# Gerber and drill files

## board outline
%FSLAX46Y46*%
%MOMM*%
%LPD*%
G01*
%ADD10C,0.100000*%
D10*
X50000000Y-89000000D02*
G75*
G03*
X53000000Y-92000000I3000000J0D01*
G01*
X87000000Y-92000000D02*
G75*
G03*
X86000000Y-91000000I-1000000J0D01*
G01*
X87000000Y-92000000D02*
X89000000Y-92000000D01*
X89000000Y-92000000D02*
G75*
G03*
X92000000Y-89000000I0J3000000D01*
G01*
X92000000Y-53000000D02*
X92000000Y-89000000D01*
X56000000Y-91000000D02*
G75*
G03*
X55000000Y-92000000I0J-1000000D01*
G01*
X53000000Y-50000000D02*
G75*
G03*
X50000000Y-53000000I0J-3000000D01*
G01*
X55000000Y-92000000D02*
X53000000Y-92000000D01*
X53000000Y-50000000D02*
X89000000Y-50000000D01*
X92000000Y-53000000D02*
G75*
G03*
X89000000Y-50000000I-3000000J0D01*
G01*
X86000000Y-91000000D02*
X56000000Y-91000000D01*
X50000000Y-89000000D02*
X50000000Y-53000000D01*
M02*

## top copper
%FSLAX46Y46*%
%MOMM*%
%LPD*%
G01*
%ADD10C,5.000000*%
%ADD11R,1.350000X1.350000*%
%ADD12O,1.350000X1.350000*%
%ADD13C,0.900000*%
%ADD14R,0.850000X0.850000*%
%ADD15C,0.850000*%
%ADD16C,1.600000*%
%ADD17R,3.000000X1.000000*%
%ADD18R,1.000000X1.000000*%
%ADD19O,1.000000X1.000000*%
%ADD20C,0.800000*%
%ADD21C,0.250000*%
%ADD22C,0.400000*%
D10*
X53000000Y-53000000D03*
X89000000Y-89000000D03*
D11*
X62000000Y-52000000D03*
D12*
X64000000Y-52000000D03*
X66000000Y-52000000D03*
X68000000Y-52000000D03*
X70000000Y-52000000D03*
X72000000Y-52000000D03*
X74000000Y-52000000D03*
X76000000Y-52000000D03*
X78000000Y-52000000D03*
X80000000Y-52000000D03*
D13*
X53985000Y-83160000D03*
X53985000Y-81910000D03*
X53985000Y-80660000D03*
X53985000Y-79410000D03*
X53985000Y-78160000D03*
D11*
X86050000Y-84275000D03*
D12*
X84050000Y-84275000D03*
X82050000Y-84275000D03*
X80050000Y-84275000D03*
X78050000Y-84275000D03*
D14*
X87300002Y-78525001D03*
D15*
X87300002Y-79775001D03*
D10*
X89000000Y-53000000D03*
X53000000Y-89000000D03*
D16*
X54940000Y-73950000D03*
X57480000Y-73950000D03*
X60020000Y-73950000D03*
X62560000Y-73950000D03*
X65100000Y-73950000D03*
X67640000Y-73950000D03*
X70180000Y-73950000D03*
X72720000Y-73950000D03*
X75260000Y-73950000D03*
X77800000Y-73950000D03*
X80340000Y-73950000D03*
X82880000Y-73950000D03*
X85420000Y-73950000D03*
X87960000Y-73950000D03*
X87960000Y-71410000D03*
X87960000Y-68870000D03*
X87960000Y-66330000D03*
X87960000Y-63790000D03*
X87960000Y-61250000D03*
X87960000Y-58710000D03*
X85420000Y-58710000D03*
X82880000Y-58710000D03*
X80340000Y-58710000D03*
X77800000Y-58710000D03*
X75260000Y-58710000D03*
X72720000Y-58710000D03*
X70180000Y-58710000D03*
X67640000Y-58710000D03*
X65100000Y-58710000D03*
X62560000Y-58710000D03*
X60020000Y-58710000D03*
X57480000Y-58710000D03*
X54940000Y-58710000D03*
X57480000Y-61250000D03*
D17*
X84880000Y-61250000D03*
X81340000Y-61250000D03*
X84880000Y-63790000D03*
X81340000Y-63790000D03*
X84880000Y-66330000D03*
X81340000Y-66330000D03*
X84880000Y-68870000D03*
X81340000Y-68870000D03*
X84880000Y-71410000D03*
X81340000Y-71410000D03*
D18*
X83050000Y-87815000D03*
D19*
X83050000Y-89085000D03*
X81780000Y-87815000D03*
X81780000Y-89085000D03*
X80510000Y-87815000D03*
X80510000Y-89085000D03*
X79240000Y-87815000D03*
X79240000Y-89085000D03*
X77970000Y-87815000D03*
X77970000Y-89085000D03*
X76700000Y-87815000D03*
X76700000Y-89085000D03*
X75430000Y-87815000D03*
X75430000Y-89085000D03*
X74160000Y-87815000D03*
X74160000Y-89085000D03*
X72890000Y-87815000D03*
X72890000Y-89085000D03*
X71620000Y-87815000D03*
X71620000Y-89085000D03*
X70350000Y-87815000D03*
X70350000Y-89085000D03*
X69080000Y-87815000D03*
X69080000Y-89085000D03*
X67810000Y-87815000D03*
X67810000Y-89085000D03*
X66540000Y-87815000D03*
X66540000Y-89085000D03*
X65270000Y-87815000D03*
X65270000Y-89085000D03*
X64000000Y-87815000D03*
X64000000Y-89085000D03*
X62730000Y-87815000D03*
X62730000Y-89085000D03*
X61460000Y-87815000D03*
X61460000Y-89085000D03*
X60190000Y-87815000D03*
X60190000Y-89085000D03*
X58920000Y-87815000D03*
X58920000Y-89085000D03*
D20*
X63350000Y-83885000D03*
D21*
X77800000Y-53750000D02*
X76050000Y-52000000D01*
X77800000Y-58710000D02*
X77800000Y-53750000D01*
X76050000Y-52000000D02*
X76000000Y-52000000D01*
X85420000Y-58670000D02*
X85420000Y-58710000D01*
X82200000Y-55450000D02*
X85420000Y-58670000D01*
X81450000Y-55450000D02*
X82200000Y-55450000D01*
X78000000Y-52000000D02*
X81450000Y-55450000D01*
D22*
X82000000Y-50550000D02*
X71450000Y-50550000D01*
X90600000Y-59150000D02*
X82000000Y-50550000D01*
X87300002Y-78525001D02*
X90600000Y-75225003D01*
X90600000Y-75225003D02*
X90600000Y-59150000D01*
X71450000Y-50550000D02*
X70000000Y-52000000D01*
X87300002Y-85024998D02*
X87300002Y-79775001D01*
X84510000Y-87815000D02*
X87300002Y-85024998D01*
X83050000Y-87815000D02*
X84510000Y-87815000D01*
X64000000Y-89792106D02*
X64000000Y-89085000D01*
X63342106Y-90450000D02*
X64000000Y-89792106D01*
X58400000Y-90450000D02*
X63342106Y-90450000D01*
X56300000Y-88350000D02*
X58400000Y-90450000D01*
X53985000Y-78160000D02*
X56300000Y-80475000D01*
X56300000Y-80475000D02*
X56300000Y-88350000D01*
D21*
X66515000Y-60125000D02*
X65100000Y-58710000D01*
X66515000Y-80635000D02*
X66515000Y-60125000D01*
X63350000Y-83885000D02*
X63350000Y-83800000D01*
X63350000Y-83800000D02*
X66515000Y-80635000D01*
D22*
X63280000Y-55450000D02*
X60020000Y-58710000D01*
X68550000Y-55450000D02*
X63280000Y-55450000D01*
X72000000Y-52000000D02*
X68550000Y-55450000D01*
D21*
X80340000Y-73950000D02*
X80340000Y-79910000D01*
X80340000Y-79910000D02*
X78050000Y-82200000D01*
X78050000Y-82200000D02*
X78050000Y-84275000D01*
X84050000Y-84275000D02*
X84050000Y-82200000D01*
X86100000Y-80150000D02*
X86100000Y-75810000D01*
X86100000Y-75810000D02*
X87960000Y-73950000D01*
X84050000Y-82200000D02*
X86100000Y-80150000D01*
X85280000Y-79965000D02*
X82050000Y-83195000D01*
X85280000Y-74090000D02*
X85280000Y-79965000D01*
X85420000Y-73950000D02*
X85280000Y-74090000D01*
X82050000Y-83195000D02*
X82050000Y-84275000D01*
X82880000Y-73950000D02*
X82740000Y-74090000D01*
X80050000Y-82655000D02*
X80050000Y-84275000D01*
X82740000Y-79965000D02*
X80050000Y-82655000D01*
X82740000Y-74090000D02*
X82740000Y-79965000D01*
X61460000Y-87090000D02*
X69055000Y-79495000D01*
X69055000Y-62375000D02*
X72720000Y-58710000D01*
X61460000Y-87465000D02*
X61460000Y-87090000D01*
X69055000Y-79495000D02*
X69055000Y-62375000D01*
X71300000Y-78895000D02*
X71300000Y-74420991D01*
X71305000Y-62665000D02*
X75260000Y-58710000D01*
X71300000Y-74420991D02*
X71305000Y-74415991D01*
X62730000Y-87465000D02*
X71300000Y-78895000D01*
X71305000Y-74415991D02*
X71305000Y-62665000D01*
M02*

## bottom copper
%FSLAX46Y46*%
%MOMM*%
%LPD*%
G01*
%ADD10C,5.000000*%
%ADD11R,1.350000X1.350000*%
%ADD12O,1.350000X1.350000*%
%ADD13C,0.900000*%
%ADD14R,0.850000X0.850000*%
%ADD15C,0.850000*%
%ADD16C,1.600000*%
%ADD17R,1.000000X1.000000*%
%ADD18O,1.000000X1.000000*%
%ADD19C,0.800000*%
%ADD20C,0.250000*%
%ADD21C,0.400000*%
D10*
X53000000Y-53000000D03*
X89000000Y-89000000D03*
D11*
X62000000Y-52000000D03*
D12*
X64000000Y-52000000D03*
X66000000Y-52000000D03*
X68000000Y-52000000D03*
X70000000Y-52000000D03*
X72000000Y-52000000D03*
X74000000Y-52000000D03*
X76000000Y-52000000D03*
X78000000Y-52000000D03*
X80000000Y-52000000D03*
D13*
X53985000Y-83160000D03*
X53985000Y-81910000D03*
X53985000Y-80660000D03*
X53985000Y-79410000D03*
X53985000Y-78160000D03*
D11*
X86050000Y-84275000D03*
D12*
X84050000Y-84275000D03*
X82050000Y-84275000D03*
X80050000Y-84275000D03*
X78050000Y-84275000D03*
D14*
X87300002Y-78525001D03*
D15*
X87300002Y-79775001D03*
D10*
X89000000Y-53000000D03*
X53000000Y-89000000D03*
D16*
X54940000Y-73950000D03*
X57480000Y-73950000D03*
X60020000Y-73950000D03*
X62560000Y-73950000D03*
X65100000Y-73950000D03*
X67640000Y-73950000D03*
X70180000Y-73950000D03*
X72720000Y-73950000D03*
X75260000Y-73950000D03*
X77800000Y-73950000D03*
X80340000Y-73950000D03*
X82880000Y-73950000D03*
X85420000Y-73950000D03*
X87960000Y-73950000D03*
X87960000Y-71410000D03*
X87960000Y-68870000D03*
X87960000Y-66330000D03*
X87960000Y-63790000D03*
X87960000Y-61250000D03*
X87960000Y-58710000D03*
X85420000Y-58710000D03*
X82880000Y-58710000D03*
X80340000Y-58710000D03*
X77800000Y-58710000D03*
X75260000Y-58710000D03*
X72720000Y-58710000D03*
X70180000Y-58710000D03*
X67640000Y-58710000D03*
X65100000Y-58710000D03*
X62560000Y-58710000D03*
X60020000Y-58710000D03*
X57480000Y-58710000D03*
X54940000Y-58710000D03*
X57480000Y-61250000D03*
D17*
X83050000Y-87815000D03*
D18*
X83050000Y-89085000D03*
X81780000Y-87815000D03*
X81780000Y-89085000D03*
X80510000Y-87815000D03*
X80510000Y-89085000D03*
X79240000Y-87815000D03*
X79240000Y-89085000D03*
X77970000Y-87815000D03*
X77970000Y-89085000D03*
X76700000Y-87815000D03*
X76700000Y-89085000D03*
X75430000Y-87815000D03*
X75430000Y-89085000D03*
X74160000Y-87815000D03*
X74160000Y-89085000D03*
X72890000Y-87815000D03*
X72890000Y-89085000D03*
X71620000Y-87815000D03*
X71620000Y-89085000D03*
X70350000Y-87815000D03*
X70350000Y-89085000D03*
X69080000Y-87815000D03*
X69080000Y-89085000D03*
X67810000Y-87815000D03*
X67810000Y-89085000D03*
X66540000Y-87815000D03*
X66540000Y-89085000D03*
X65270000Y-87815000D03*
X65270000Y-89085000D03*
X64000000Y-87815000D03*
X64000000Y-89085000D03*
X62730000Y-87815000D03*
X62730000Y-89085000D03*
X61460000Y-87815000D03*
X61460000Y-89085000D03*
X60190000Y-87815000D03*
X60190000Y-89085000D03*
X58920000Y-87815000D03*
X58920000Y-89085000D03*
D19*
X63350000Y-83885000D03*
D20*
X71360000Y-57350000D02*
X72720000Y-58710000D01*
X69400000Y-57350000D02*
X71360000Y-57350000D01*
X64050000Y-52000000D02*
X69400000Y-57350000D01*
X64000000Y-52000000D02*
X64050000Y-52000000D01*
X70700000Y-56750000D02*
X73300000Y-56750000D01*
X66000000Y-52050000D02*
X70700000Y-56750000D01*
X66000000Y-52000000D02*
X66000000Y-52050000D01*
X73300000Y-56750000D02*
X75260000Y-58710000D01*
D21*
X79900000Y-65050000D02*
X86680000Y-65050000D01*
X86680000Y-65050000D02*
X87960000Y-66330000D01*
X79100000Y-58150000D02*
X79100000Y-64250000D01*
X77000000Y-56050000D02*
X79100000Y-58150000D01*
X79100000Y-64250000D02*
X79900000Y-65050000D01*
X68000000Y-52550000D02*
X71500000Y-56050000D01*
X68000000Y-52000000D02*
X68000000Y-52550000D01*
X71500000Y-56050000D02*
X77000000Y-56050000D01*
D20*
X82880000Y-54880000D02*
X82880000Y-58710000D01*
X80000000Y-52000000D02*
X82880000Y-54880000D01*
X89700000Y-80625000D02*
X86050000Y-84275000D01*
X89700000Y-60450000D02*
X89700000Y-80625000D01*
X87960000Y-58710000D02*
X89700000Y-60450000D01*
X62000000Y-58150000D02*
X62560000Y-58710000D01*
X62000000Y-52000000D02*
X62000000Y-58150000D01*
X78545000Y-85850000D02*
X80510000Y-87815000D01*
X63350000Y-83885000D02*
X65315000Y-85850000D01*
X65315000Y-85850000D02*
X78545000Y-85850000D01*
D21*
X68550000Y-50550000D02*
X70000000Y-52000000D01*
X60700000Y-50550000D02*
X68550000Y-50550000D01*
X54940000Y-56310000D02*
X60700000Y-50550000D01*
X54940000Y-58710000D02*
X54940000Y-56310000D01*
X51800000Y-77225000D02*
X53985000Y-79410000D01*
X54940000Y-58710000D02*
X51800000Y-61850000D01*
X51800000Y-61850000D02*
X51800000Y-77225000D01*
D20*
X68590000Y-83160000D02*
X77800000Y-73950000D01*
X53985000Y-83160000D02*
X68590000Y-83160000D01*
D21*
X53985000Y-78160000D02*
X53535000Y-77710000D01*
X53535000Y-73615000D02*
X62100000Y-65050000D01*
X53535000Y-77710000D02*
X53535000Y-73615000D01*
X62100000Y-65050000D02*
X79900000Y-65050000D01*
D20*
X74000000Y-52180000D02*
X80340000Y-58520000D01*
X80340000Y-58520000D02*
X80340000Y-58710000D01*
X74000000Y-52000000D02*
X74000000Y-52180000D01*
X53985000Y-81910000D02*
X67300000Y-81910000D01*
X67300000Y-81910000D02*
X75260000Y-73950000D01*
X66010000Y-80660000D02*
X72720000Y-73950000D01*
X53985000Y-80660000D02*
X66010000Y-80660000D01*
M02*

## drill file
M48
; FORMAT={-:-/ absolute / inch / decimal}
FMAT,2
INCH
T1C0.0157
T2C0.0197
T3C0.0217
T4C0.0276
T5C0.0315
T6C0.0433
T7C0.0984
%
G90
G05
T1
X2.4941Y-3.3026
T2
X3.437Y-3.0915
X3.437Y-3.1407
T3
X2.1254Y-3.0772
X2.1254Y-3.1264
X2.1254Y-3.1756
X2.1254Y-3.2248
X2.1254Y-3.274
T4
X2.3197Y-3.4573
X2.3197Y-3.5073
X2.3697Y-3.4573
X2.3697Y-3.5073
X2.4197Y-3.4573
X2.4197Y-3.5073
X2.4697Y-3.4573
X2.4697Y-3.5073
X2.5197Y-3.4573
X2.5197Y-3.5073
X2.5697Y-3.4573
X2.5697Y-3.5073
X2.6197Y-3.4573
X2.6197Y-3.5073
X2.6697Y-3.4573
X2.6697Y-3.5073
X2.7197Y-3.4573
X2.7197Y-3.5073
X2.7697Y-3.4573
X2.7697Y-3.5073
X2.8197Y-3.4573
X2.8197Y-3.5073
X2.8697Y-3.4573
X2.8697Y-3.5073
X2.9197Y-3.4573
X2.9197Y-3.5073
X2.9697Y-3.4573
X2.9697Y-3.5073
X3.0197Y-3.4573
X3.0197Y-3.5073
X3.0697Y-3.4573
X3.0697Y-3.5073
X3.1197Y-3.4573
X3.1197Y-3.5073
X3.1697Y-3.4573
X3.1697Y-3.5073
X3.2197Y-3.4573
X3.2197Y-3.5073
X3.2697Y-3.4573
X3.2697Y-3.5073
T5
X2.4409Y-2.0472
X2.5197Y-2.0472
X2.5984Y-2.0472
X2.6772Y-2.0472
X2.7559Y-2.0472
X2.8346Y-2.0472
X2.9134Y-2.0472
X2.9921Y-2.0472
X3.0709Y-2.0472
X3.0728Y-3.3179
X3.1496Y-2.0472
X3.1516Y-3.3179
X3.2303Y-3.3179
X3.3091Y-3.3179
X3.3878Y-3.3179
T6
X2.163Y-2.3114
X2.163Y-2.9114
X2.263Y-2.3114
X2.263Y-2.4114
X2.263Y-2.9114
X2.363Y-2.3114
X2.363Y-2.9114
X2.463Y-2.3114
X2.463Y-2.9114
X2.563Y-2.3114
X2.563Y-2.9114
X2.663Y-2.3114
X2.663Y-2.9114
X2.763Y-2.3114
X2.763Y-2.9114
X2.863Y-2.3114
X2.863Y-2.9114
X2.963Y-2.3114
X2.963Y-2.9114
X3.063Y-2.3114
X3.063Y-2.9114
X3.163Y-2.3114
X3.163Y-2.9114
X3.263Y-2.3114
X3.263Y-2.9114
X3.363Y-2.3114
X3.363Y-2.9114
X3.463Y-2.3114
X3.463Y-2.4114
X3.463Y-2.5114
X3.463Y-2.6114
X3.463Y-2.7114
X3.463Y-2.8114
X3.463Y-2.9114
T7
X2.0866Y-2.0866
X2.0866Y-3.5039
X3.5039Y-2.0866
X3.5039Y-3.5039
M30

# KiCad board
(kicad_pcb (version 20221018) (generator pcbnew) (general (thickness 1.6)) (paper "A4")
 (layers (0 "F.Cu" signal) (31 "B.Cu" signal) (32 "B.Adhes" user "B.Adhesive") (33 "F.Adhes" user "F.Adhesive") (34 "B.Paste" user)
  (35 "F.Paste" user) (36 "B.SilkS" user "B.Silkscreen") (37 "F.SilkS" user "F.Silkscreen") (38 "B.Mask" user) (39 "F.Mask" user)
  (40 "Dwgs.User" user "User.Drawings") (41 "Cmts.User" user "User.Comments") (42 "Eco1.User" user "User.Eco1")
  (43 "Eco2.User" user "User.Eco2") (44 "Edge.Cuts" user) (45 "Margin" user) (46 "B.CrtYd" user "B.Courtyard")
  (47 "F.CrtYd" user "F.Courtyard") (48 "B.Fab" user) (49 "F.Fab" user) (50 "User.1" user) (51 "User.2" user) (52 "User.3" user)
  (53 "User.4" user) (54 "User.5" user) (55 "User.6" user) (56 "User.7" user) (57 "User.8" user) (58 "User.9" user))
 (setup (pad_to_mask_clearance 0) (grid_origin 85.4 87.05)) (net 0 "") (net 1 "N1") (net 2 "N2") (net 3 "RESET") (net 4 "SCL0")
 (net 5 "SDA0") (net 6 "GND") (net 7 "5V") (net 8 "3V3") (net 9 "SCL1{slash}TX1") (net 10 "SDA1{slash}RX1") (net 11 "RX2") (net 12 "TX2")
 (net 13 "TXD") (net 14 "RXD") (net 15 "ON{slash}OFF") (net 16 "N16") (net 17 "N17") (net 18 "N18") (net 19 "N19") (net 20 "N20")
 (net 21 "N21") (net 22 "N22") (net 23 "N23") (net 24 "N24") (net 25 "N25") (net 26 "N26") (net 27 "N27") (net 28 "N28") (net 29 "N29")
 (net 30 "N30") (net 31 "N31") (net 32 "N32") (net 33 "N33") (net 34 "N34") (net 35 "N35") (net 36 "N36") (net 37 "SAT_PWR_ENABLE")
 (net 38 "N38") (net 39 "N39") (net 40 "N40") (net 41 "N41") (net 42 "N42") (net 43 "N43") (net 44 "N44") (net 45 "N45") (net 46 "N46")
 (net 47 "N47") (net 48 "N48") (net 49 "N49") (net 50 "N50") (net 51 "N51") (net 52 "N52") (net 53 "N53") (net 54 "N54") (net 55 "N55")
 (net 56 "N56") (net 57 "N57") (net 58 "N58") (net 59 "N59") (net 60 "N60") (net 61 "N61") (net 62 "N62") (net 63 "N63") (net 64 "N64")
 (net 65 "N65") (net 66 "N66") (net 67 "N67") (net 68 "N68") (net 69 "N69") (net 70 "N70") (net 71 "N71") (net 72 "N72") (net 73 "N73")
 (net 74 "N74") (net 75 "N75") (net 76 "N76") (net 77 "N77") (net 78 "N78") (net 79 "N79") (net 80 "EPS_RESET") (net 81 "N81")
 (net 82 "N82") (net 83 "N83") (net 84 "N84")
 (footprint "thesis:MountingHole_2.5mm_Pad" (layer "F.Cu") (at 53 53)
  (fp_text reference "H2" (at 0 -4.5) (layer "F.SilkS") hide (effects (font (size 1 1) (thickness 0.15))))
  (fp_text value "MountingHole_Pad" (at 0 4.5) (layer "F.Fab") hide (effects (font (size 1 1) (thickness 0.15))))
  (pad "1" thru_hole circle (at 0 0) (size 5 5) (drill 2.5) (layers "*.Cu" "*.Mask") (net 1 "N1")))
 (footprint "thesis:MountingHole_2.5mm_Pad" (layer "F.Cu") (at 89 89)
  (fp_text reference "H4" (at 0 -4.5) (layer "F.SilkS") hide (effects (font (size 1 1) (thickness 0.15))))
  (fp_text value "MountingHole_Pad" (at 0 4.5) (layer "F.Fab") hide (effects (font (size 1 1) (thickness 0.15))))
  (pad "1" thru_hole circle (at 0 0) (size 5 5) (drill 2.5) (layers "*.Cu" "*.Mask") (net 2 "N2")))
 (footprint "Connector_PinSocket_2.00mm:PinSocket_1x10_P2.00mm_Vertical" (layer "F.Cu") (at 62 52 90)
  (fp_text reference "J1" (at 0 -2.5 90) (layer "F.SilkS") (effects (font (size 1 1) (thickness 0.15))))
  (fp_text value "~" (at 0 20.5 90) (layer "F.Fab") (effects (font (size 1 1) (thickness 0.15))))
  (pad "1" thru_hole rect (at 0 0 90) (size 1.35 1.35) (drill 0.8) (layers "*.Cu" "*.Mask") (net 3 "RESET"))
  (pad "2" thru_hole oval (at 0 2 90) (size 1.35 1.35) (drill 0.8) (layers "*.Cu" "*.Mask") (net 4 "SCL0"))
  (pad "3" thru_hole oval (at 0 4 90) (size 1.35 1.35) (drill 0.8) (layers "*.Cu" "*.Mask") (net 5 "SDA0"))
  (pad "4" thru_hole oval (at 0 6 90) (size 1.35 1.35) (drill 0.8) (layers "*.Cu" "*.Mask") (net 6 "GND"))
  (pad "5" thru_hole oval (at 0 8 90) (size 1.35 1.35) (drill 0.8) (layers "*.Cu" "*.Mask") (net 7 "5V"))
  (pad "6" thru_hole oval (at 0 10 90) (size 1.35 1.35) (drill 0.8) (layers "*.Cu" "*.Mask") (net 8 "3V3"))
  (pad "7" thru_hole oval (at 0 12 90) (size 1.35 1.35) (drill 0.8) (layers "*.Cu" "*.Mask") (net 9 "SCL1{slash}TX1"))
  (pad "8" thru_hole oval (at 0 14 90) (size 1.35 1.35) (drill 0.8) (layers "*.Cu" "*.Mask") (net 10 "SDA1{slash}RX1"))
  (pad "9" thru_hole oval (at 0 16 90) (size 1.35 1.35) (drill 0.8) (layers "*.Cu" "*.Mask") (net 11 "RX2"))
  (pad "10" thru_hole oval (at 0 18 90) (size 1.35 1.35) (drill 0.8) (layers "*.Cu" "*.Mask") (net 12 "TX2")))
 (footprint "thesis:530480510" (layer "F.Cu") (at 57.8 76.85 -90)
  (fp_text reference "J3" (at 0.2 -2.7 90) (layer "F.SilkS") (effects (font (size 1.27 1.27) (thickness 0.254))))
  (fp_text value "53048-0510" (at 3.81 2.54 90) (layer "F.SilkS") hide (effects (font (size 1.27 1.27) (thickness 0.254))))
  (pad "1" thru_hole circle (at 6.31 3.815 270) (size 0.9 0.9) (drill 0.55) (layers "*.Cu" "*.Mask") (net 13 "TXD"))
  (pad "2" thru_hole circle (at 5.06 3.815 270) (size 0.9 0.9) (drill 0.55) (layers "*.Cu" "*.Mask") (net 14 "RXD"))
  (pad "3" thru_hole circle (at 3.81 3.815 270) (size 0.9 0.9) (drill 0.55) (layers "*.Cu" "*.Mask") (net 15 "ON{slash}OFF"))
  (pad "4" thru_hole circle (at 2.56 3.815 270) (size 0.9 0.9) (drill 0.55) (layers "*.Cu" "*.Mask") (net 7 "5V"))
  (pad "5" thru_hole circle (at 1.31 3.815 270) (size 0.9 0.9) (drill 0.55) (layers "*.Cu" "*.Mask") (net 6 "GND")))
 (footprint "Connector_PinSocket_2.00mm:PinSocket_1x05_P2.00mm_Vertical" (layer "F.Cu") (at 86.05 84.275 -90)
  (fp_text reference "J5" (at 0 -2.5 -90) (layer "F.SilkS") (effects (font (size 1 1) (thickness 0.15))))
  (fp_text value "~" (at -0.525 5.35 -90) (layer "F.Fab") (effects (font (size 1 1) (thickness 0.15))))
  (pad "1" thru_hole rect (at 0 0 270) (size 1.35 1.35) (drill 0.8) (layers "*.Cu" "*.Mask") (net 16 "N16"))
  (pad "2" thru_hole oval (at 0 2 270) (size 1.35 1.35) (drill 0.8) (layers "*.Cu" "*.Mask") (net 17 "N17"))
  (pad "3" thru_hole oval (at 0 4 270) (size 1.35 1.35) (drill 0.8) (layers "*.Cu" "*.Mask") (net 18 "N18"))
  (pad "4" thru_hole oval (at 0 6 270) (size 1.35 1.35) (drill 0.8) (layers "*.Cu" "*.Mask") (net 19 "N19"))
  (pad "5" thru_hole oval (at 0 8 270) (size 1.35 1.35) (drill 0.8) (layers "*.Cu" "*.Mask") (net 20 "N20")))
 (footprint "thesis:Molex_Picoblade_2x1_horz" (layer "F.Cu") (at 87.300002 78.525001 -90)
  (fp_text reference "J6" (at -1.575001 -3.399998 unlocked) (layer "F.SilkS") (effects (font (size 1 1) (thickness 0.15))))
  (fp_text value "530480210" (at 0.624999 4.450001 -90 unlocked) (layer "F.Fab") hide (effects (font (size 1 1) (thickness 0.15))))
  (pad "1" thru_hole rect (at 0 0 270) (size 0.85 0.85) (drill 0.5) (layers "*.Cu" "*.Mask") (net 7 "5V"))
  (pad "2" thru_hole circle (at 1.25 0 270) (size 0.85 0.85) (drill 0.5) (layers "*.Cu" "*.Mask") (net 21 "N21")))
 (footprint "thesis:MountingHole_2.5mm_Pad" (layer "F.Cu") (at 89 53)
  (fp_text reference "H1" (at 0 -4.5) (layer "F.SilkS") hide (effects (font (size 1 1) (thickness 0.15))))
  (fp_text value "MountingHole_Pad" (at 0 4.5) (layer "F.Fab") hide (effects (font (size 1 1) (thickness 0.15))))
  (pad "1" thru_hole circle (at 0 0) (size 5 5) (drill 2.5) (layers "*.Cu" "*.Mask") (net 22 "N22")))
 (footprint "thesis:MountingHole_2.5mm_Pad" (layer "F.Cu") (at 53 89)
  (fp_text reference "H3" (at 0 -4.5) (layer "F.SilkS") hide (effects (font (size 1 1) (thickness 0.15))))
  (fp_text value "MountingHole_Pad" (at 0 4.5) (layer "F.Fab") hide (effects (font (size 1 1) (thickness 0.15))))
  (pad "1" thru_hole circle (at 0 0) (size 5 5) (drill 2.5) (layers "*.Cu" "*.Mask") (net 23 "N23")))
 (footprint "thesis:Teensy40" (layer "F.Cu") (at 71.45 66.33)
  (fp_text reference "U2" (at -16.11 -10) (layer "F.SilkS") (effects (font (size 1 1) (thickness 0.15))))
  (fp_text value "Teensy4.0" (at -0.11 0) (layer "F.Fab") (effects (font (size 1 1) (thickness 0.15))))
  (pad "1" thru_hole circle (at -16.51 7.62) (size 1.6 1.6) (drill 1.1) (layers "*.Cu" "*.Mask") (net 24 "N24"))
  (pad "2" thru_hole circle (at -13.97 7.62) (size 1.6 1.6) (drill 1.1) (layers "*.Cu" "*.Mask") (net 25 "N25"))
  (pad "3" thru_hole circle (at -11.43 7.62) (size 1.6 1.6) (drill 1.1) (layers "*.Cu" "*.Mask") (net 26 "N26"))
  (pad "4" thru_hole circle (at -8.89 7.62) (size 1.6 1.6) (drill 1.1) (layers "*.Cu" "*.Mask") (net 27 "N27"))
  (pad "5" thru_hole circle (at -6.35 7.62) (size 1.6 1.6) (drill 1.1) (layers "*.Cu" "*.Mask") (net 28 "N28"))
  (pad "6" thru_hole circle (at -3.81 7.62) (size 1.6 1.6) (drill 1.1) (layers "*.Cu" "*.Mask") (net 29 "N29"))
  (pad "7" thru_hole circle (at -1.27 7.62) (size 1.6 1.6) (drill 1.1) (layers "*.Cu" "*.Mask") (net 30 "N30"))
  (pad "8" thru_hole circle (at 1.27 7.62) (size 1.6 1.6) (drill 1.1) (layers "*.Cu" "*.Mask") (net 15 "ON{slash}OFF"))
  (pad "9" thru_hole circle (at 3.81 7.62) (size 1.6 1.6) (drill 1.1) (layers "*.Cu" "*.Mask") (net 14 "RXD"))
  (pad "10" thru_hole circle (at 6.35 7.62) (size 1.6 1.6) (drill 1.1) (layers "*.Cu" "*.Mask") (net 13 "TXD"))
  (pad "11" thru_hole circle (at 8.89 7.62) (size 1.6 1.6) (drill 1.1) (layers "*.Cu" "*.Mask") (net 20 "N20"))
  (pad "12" thru_hole circle (at 11.43 7.62) (size 1.6 1.6) (drill 1.1) (layers "*.Cu" "*.Mask") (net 19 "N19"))
  (pad "13" thru_hole circle (at 13.97 7.62) (size 1.6 1.6) (drill 1.1) (layers "*.Cu" "*.Mask") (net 18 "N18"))
  (pad "14" thru_hole circle (at 16.51 7.62) (size 1.6 1.6) (drill 1.1) (layers "*.Cu" "*.Mask") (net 17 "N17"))
  (pad "15" thru_hole circle (at 16.51 5.08) (size 1.6 1.6) (drill 1.1) (layers "*.Cu" "*.Mask") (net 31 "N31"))
  (pad "16" thru_hole circle (at 16.51 2.54) (size 1.6 1.6) (drill 1.1) (layers "*.Cu" "*.Mask") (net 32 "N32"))
  (pad "17" thru_hole circle (at 16.51 0) (size 1.6 1.6) (drill 1.1) (layers "*.Cu" "*.Mask") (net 6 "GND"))
  (pad "18" thru_hole circle (at 16.51 -2.54) (size 1.6 1.6) (drill 1.1) (layers "*.Cu" "*.Mask") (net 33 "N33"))
  (pad "19" thru_hole circle (at 16.51 -5.08) (size 1.6 1.6) (drill 1.1) (layers "*.Cu" "*.Mask") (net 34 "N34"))
  (pad "20" thru_hole circle (at 16.51 -7.62) (size 1.6 1.6) (drill 1.1) (layers "*.Cu" "*.Mask") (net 16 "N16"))
  (pad "21" thru_hole circle (at 13.97 -7.62) (size 1.6 1.6) (drill 1.1) (layers "*.Cu" "*.Mask") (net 11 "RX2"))
  (pad "22" thru_hole circle (at 11.43 -7.62) (size 1.6 1.6) (drill 1.1) (layers "*.Cu" "*.Mask") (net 12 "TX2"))
  (pad "23" thru_hole circle (at 8.89 -7.62) (size 1.6 1.6) (drill 1.1) (layers "*.Cu" "*.Mask") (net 9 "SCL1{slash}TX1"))
  (pad "24" thru_hole circle (at 6.35 -7.62) (size 1.6 1.6) (drill 1.1) (layers "*.Cu" "*.Mask") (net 10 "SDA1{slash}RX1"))
  (pad "25" thru_hole circle (at 3.81 -7.62) (size 1.6 1.6) (drill 1.1) (layers "*.Cu" "*.Mask") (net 5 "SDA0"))
  (pad "26" thru_hole circle (at 1.27 -7.62) (size 1.6 1.6) (drill 1.1) (layers "*.Cu" "*.Mask") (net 4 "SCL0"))
  (pad "27" thru_hole circle (at -1.27 -7.62) (size 1.6 1.6) (drill 1.1) (layers "*.Cu" "*.Mask") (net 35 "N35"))
  (pad "28" thru_hole circle (at -3.81 -7.62) (size 1.6 1.6) (drill 1.1) (layers "*.Cu" "*.Mask") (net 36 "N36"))
  (pad "29" thru_hole circle (at -6.35 -7.62) (size 1.6 1.6) (drill 1.1) (layers "*.Cu" "*.Mask") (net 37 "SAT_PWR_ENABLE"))
  (pad "30" thru_hole circle (at -8.89 -7.62) (size 1.6 1.6) (drill 1.1) (layers "*.Cu" "*.Mask") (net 3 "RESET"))
  (pad "31" thru_hole circle (at -11.43 -7.62) (size 1.6 1.6) (drill 1.1) (layers "*.Cu" "*.Mask") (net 8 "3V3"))
  (pad "32" thru_hole circle (at -13.97 -7.62) (size 1.6 1.6) (drill 1.1) (layers "*.Cu" "*.Mask") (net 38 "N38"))
  (pad "33" thru_hole circle (at -16.51 -7.62) (size 1.6 1.6) (drill 1.1) (layers "*.Cu" "*.Mask") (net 7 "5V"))
  (pad "34" thru_hole circle (at -13.97 -5.08) (size 1.6 1.6) (drill 1.1) (layers "*.Cu" "*.Mask") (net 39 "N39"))
  (pad "35" smd rect (at 13.43 -5.08) (size 3 1) (layers "F.Cu" "F.Paste" "F.Mask") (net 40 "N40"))
  (pad "36" smd rect (at 9.89 -5.08) (size 3 1) (layers "F.Cu" "F.Paste" "F.Mask") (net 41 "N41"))
  (pad "37" smd rect (at 13.43 -2.54) (size 3 1) (layers "F.Cu" "F.Paste" "F.Mask") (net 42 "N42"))
  (pad "38" smd rect (at 9.89 -2.54) (size 3 1) (layers "F.Cu" "F.Paste" "F.Mask") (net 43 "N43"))
  (pad "39" smd rect (at 13.43 0) (size 3 1) (layers "F.Cu" "F.Paste" "F.Mask") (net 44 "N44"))
  (pad "40" smd rect (at 9.89 0) (size 3 1) (layers "F.Cu" "F.Paste" "F.Mask") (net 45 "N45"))
  (pad "41" smd rect (at 13.43 2.54) (size 3 1) (layers "F.Cu" "F.Paste" "F.Mask") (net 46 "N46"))
  (pad "42" smd rect (at 9.89 2.54) (size 3 1) (layers "F.Cu" "F.Paste" "F.Mask") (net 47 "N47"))
  (pad "43" smd rect (at 13.43 5.08) (size 3 1) (layers "F.Cu" "F.Paste" "F.Mask") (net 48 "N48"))
  (pad "44" smd rect (at 9.89 5.08) (size 3 1) (layers "F.Cu" "F.Paste" "F.Mask") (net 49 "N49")))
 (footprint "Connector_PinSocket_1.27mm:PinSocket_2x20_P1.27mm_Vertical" (layer "B.Cu") (at 60.19 89.355 -90)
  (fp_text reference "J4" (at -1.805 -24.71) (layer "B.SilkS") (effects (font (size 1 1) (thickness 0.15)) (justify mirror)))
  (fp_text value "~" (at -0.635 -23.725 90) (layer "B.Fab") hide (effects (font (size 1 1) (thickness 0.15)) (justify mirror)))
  (pad "1" thru_hole rect (at -1.54 -22.86 270) (size 1 1) (drill 0.7) (layers "*.Cu" "*.Mask") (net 21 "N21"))
  (pad "2" thru_hole oval (at -0.27 -22.86 270) (size 1 1) (drill 0.7) (layers "*.Cu" "*.Mask") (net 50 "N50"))
  (pad "3" thru_hole oval (at -1.54 -21.59 270) (size 1 1) (drill 0.7) (layers "*.Cu" "*.Mask") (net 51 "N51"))
  (pad "4" thru_hole oval (at -0.27 -21.59 270) (size 1 1) (drill 0.7) (layers "*.Cu" "*.Mask") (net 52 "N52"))
  (pad "5" thru_hole oval (at -1.54 -20.32 270) (size 1 1) (drill 0.7) (layers "*.Cu" "*.Mask") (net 37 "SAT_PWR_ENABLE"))
  (pad "6" thru_hole oval (at -0.27 -20.32 270) (size 1 1) (drill 0.7) (layers "*.Cu" "*.Mask") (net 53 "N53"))
  (pad "7" thru_hole oval (at -1.54 -19.05 270) (size 1 1) (drill 0.7) (layers "*.Cu" "*.Mask") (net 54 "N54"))
  (pad "8" thru_hole oval (at -0.27 -19.05 270) (size 1 1) (drill 0.7) (layers "*.Cu" "*.Mask") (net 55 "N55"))
  (pad "9" thru_hole oval (at -1.54 -17.78 270) (size 1 1) (drill 0.7) (layers "*.Cu" "*.Mask") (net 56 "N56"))
  (pad "10" thru_hole oval (at -0.27 -17.78 270) (size 1 1) (drill 0.7) (layers "*.Cu" "*.Mask") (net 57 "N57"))
  (pad "11" thru_hole oval (at -1.54 -16.51 270) (size 1 1) (drill 0.7) (layers "*.Cu" "*.Mask") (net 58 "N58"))
  (pad "12" thru_hole oval (at -0.27 -16.51 270) (size 1 1) (drill 0.7) (layers "*.Cu" "*.Mask") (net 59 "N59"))
  (pad "13" thru_hole oval (at -1.54 -15.24 270) (size 1 1) (drill 0.7) (layers "*.Cu" "*.Mask") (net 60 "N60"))
  (pad "14" thru_hole oval (at -0.27 -15.24 270) (size 1 1) (drill 0.7) (layers "*.Cu" "*.Mask") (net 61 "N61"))
  (pad "15" thru_hole oval (at -1.54 -13.97 270) (size 1 1) (drill 0.7) (layers "*.Cu" "*.Mask") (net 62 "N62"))
  (pad "16" thru_hole oval (at -0.27 -13.97 270) (size 1 1) (drill 0.7) (layers "*.Cu" "*.Mask") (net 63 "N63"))
  (pad "17" thru_hole oval (at -1.54 -12.7 270) (size 1 1) (drill 0.7) (layers "*.Cu" "*.Mask") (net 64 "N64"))
  (pad "18" thru_hole oval (at -0.27 -12.7 270) (size 1 1) (drill 0.7) (layers "*.Cu" "*.Mask") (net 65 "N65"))
  (pad "19" thru_hole oval (at -1.54 -11.43 270) (size 1 1) (drill 0.7) (layers "*.Cu" "*.Mask") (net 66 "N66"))
  (pad "20" thru_hole oval (at -0.27 -11.43 270) (size 1 1) (drill 0.7) (layers "*.Cu" "*.Mask") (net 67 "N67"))
  (pad "21" thru_hole oval (at -1.54 -10.16 270) (size 1 1) (drill 0.7) (layers "*.Cu" "*.Mask") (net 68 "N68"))
  (pad "22" thru_hole oval (at -0.27 -10.16 270) (size 1 1) (drill 0.7) (layers "*.Cu" "*.Mask") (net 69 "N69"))
  (pad "23" thru_hole oval (at -1.54 -8.89 270) (size 1 1) (drill 0.7) (layers "*.Cu" "*.Mask") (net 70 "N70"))
  (pad "24" thru_hole oval (at -0.27 -8.89 270) (size 1 1) (drill 0.7) (layers "*.Cu" "*.Mask") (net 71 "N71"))
  (pad "25" thru_hole oval (at -1.54 -7.62 270) (size 1 1) (drill 0.7) (layers "*.Cu" "*.Mask") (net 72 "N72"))
  (pad "26" thru_hole oval (at -0.27 -7.62 270) (size 1 1) (drill 0.7) (layers "*.Cu" "*.Mask") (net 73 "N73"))
  (pad "27" thru_hole oval (at -1.54 -6.35 270) (size 1 1) (drill 0.7) (layers "*.Cu" "*.Mask") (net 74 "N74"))
  (pad "28" thru_hole oval (at -0.27 -6.35 270) (size 1 1) (drill 0.7) (layers "*.Cu" "*.Mask") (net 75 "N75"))
  (pad "29" thru_hole oval (at -1.54 -5.08 270) (size 1 1) (drill 0.7) (layers "*.Cu" "*.Mask") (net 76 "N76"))
  (pad "30" thru_hole oval (at -0.27 -5.08 270) (size 1 1) (drill 0.7) (layers "*.Cu" "*.Mask") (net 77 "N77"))
  (pad "31" thru_hole oval (at -1.54 -3.81 270) (size 1 1) (drill 0.7) (layers "*.Cu" "*.Mask") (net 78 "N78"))
  (pad "32" thru_hole oval (at -0.27 -3.81 270) (size 1 1) (drill 0.7) (layers "*.Cu" "*.Mask") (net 6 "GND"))
  (pad "33" thru_hole oval (at -1.54 -2.54 270) (size 1 1) (drill 0.7) (layers "*.Cu" "*.Mask") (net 5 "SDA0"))
  (pad "34" thru_hole oval (at -0.27 -2.54 270) (size 1 1) (drill 0.7) (layers "*.Cu" "*.Mask") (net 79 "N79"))
  (pad "35" thru_hole oval (at -1.54 -1.27 270) (size 1 1) (drill 0.7) (layers "*.Cu" "*.Mask") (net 4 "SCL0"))
  (pad "36" thru_hole oval (at -0.27 -1.27 270) (size 1 1) (drill 0.7) (layers "*.Cu" "*.Mask") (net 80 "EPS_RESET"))
  (pad "37" thru_hole oval (at -1.54 0 270) (size 1 1) (drill 0.7) (layers "*.Cu" "*.Mask") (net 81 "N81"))
  (pad "38" thru_hole oval (at -0.27 0 270) (size 1 1) (drill 0.7) (layers "*.Cu" "*.Mask") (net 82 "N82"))
  (pad "39" thru_hole oval (at -1.54 1.27 270) (size 1 1) (drill 0.7) (layers "*.Cu" "*.Mask") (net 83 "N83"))
  (pad "40" thru_hole oval (at -0.27 1.27 270) (size 1 1) (drill 0.7) (layers "*.Cu" "*.Mask") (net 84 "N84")))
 (gr_arc (start 53 92) (mid 50.87868 91.12132) (end 50 89) (stroke (width 0.1) (type default)) (layer "Edge.Cuts"))
 (gr_arc (start 86 91) (mid 86.707107 91.292893) (end 87 92) (stroke (width 0.1) (type default)) (layer "Edge.Cuts"))
 (gr_line (start 87 92) (end 89 92) (stroke (width 0.1) (type default)) (layer "Edge.Cuts"))
 (gr_arc (start 92 89) (mid 91.12132 91.12132) (end 89 92) (stroke (width 0.1) (type default)) (layer "Edge.Cuts"))
 (gr_line (start 92 53) (end 92 89) (stroke (width 0.1) (type default)) (layer "Edge.Cuts"))
 (gr_arc (start 55 92) (mid 55.292893 91.292893) (end 56 91) (stroke (width 0.1) (type default)) (layer "Edge.Cuts"))
 (gr_arc (start 50 53) (mid 50.87868 50.87868) (end 53 50) (stroke (width 0.1) (type default)) (layer "Edge.Cuts"))
 (gr_line (start 55 92) (end 53 92) (stroke (width 0.1) (type default)) (layer "Edge.Cuts"))
 (gr_line (start 53 50) (end 89 50) (stroke (width 0.1) (type default)) (layer "Edge.Cuts"))
 (gr_arc (start 89 50) (mid 91.12132 50.87868) (end 92 53) (stroke (width 0.1) (type default)) (layer "Edge.Cuts"))
 (gr_line (start 86 91) (end 56 91) (stroke (width 0.1) (type default)) (layer "Edge.Cuts"))
 (gr_line (start 50 89) (end 50 53) (stroke (width 0.1) (type default)) (layer "Edge.Cuts"))
 (segment (start 71.45 50.55) (end 70 52) (width 0.4) (layer "F.Cu") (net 7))
 (segment (start 90.6 59.15) (end 82 50.55) (width 0.4) (layer "F.Cu") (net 7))
 (segment (start 90.6 75.225003) (end 90.6 59.15) (width 0.4) (layer "F.Cu") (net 7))
 (segment (start 82 50.55) (end 71.45 50.55) (width 0.4) (layer "F.Cu") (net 7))
 (segment (start 87.300002 78.525001) (end 90.6 75.225003) (width 0.4) (layer "F.Cu") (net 7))
 (segment (start 54.94 56.31) (end 60.7 50.55) (width 0.4) (layer "B.Cu") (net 7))
 (segment (start 68.55 50.55) (end 70 52) (width 0.4) (layer "B.Cu") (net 7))
 (segment (start 60.7 50.55) (end 68.55 50.55) (width 0.4) (layer "B.Cu") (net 7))
 (segment (start 51.8 77.225) (end 53.985 79.41) (width 0.4) (layer "B.Cu") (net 7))
 (segment (start 54.94 58.71) (end 54.94 56.31) (width 0.4) (layer "B.Cu") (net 7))
 (segment (start 54.94 58.71) (end 51.8 61.85) (width 0.4) (layer "B.Cu") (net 7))
 (segment (start 51.8 61.85) (end 51.8 77.225) (width 0.4) (layer "B.Cu") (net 7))
 (segment (start 63.28 55.45) (end 60.02 58.71) (width 0.4) (layer "F.Cu") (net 8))
 (segment (start 72 52) (end 68.55 55.45) (width 0.4) (layer "F.Cu") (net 8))
 (segment (start 68.55 55.45) (end 63.28 55.45) (width 0.4) (layer "F.Cu") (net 8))
 (segment (start 80.34 73.95) (end 80.34 79.91) (width 0.25) (layer "F.Cu") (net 20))
 (segment (start 80.34 79.91) (end 78.05 82.2) (width 0.25) (layer "F.Cu") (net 20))
 (segment (start 78.05 82.2) (end 78.05 84.275) (width 0.25) (layer "F.Cu") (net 20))
 (segment (start 89.7 80.625) (end 86.05 84.275) (width 0.25) (layer "B.Cu") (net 16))
 (segment (start 87.96 58.71) (end 89.7 60.45) (width 0.25) (layer "B.Cu") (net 16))
 (segment (start 89.7 60.45) (end 89.7 80.625) (width 0.25) (layer "B.Cu") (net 16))
 (segment (start 84.05 84.275) (end 84.05 82.2) (width 0.25) (layer "F.Cu") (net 17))
 (segment (start 86.1 80.15) (end 86.1 75.81) (width 0.25) (layer "F.Cu") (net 17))
 (segment (start 86.1 75.81) (end 87.96 73.95) (width 0.25) (layer "F.Cu") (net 17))
 (segment (start 84.05 82.2) (end 86.1 80.15) (width 0.25) (layer "F.Cu") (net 17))
 (segment (start 85.28 79.965) (end 82.05 83.195) (width 0.25) (layer "F.Cu") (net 18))
 (segment (start 85.28 74.09) (end 85.28 79.965) (width 0.25) (layer "F.Cu") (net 18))
 (segment (start 85.42 73.95) (end 85.28 74.09) (width 0.25) (layer "F.Cu") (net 18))
 (segment (start 82.05 83.195) (end 82.05 84.275) (width 0.25) (layer "F.Cu") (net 18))
 (segment (start 82.88 73.95) (end 82.74 74.09) (width 0.25) (layer "F.Cu") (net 19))
 (segment (start 80.05 82.655) (end 80.05 84.275) (width 0.25) (layer "F.Cu") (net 19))
 (segment (start 82.74 79.965) (end 80.05 82.655) (width 0.25) (layer "F.Cu") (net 19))
 (segment (start 82.74 74.09) (end 82.74 79.965) (width 0.25) (layer "F.Cu") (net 19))
 (segment (start 53.985 81.91) (end 67.3 81.91) (width 0.25) (layer "B.Cu") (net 14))
 (segment (start 67.3 81.91) (end 75.26 73.95) (width 0.25) (layer "B.Cu") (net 14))
 (segment (start 61.46 87.09) (end 69.055 79.495) (width 0.25) (layer "F.Cu") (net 4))
 (segment (start 69.055 62.375) (end 72.72 58.71) (width 0.25) (layer "F.Cu") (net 4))
 (segment (start 61.46 87.465) (end 61.46 87.09) (width 0.25) (layer "F.Cu") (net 4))
 (segment (start 69.055 79.495) (end 69.055 62.375) (width 0.25) (layer "F.Cu") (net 4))
 (segment (start 69.4 57.35) (end 71.36 57.35) (width 0.25) (layer "B.Cu") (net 4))
 (segment (start 64 52) (end 64.05 52) (width 0.25) (layer "B.Cu") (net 4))
 (segment (start 64.05 52) (end 69.4 57.35) (width 0.25) (layer "B.Cu") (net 4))
 (segment (start 71.36 57.35) (end 72.72 58.71) (width 0.25) (layer "B.Cu") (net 4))
 (segment (start 71.3 78.895) (end 71.3 74.420991) (width 0.25) (layer "F.Cu") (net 5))
 (segment (start 71.305 62.665) (end 75.26 58.71) (width 0.25) (layer "F.Cu") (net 5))
 (segment (start 71.3 74.420991) (end 71.305 74.415991) (width 0.25) (layer "F.Cu") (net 5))
 (segment (start 62.73 87.465) (end 71.3 78.895) (width 0.25) (layer "F.Cu") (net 5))
 (segment (start 71.305 74.415991) (end 71.305 62.665) (width 0.25) (layer "F.Cu") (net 5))
 (segment (start 66 52.05) (end 70.7 56.75) (width 0.25) (layer "B.Cu") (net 5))
 (segment (start 73.3 56.75) (end 75.26 58.71) (width 0.25) (layer "B.Cu") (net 5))
 (segment (start 70.7 56.75) (end 73.3 56.75) (width 0.25) (layer "B.Cu") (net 5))
 (segment (start 66 52) (end 66 52.05) (width 0.25) (layer "B.Cu") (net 5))
 (segment (start 58.4 90.45) (end 63.342106 90.45) (width 0.4) (layer "F.Cu") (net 6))
 (segment (start 56.3 88.35) (end 58.4 90.45) (width 0.4) (layer "F.Cu") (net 6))
 (segment (start 64 89.792106) (end 64 89.085) (width 0.4) (layer "F.Cu") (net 6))
 (segment (start 63.342106 90.45) (end 64 89.792106) (width 0.4) (layer "F.Cu") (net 6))
 (segment (start 53.985 78.16) (end 56.3 80.475) (width 0.4) (layer "F.Cu") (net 6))
 (segment (start 56.3 80.475) (end 56.3 88.35) (width 0.4) (layer "F.Cu") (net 6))
 (segment (start 53.985 78.16) (end 53.535 77.71) (width 0.4) (layer "B.Cu") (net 6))
 (segment (start 79.1 64.25) (end 79.9 65.05) (width 0.4) (layer "B.Cu") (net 6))
 (segment (start 79.1 58.15) (end 79.1 64.25) (width 0.4) (layer "B.Cu") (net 6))
 (segment (start 53.535 73.615) (end 62.1 65.05) (width 0.4) (layer "B.Cu") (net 6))
 (segment (start 53.535 77.71) (end 53.535 73.615) (width 0.4) (layer "B.Cu") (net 6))
 (segment (start 68 52) (end 68 52.55) (width 0.4) (layer "B.Cu") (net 6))
 (segment (start 68 52.55) (end 71.5 56.05) (width 0.4) (layer "B.Cu") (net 6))
 (segment (start 77 56.05) (end 79.1 58.15) (width 0.4) (layer "B.Cu") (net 6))
 (segment (start 79.9 65.05) (end 86.68 65.05) (width 0.4) (layer "B.Cu") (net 6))
 (segment (start 71.5 56.05) (end 77 56.05) (width 0.4) (layer "B.Cu") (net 6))
 (segment (start 62.1 65.05) (end 79.9 65.05) (width 0.4) (layer "B.Cu") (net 6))
 (segment (start 86.68 65.05) (end 87.96 66.33) (width 0.4) (layer "B.Cu") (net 6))
 (segment (start 74 52.18) (end 80.34 58.52) (width 0.25) (layer "B.Cu") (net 9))
 (segment (start 80.34 58.52) (end 80.34 58.71) (width 0.25) (layer "B.Cu") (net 9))
 (segment (start 74 52) (end 74 52.18) (width 0.25) (layer "B.Cu") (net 9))
 (segment (start 76.05 52) (end 76 52) (width 0.25) (layer "F.Cu") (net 10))
 (segment (start 77.8 53.75) (end 76.05 52) (width 0.25) (layer "F.Cu") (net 10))
 (segment (start 77.8 58.71) (end 77.8 53.75) (width 0.25) (layer "F.Cu") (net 10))
 (segment (start 85.42 58.67) (end 85.42 58.71) (width 0.25) (layer "F.Cu") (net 11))
 (segment (start 81.45 55.45) (end 82.2 55.45) (width 0.25) (layer "F.Cu") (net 11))
 (segment (start 78 52) (end 81.45 55.45) (width 0.25) (layer "F.Cu") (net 11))
 (segment (start 82.2 55.45) (end 85.42 58.67) (width 0.25) (layer "F.Cu") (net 11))
 (segment (start 82.88 54.88) (end 82.88 58.71) (width 0.25) (layer "B.Cu") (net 12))
 (segment (start 80 52) (end 82.88 54.88) (width 0.25) (layer "B.Cu") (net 12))
 (segment (start 66.515 60.125) (end 65.1 58.71) (width 0.25) (layer "F.Cu") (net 37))
 (segment (start 63.35 83.8) (end 66.515 80.635) (width 0.25) (layer "F.Cu") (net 37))
 (segment (start 63.35 83.885) (end 63.35 83.8) (width 0.25) (layer "F.Cu") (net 37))
 (segment (start 66.515 80.635) (end 66.515 60.125) (width 0.25) (layer "F.Cu") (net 37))
 (via (at 63.35 83.885) (size 0.8) (drill 0.4) (layers "F.Cu" "B.Cu") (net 37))
 (segment (start 78.545 85.85) (end 80.51 87.815) (width 0.25) (layer "B.Cu") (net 37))
 (segment (start 65.315 85.85) (end 78.545 85.85) (width 0.25) (layer "B.Cu") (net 37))
 (segment (start 63.35 83.885) (end 65.315 85.85) (width 0.25) (layer "B.Cu") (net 37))
 (segment (start 84.51 87.815) (end 87.300002 85.024998) (width 0.4) (layer "F.Cu") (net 21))
 (segment (start 83.05 87.815) (end 84.51 87.815) (width 0.4) (layer "F.Cu") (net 21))
 (segment (start 87.300002 85.024998) (end 87.300002 79.775001) (width 0.4) (layer "F.Cu") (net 21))
 (segment (start 68.59 83.16) (end 77.8 73.95) (width 0.25) (layer "B.Cu") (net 13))
 (segment (start 53.985 83.16) (end 68.59 83.16) (width 0.25) (layer "B.Cu") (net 13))
 (segment (start 66.01 80.66) (end 72.72 73.95) (width 0.25) (layer "B.Cu") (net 15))
 (segment (start 53.985 80.66) (end 66.01 80.66) (width 0.25) (layer "B.Cu") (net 15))
 (segment (start 62 58.15) (end 62.56 58.71) (width 0.25) (layer "B.Cu") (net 3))
 (segment (start 62 52) (end 62 58.15) (width 0.25) (layer "B.Cu") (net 3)))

